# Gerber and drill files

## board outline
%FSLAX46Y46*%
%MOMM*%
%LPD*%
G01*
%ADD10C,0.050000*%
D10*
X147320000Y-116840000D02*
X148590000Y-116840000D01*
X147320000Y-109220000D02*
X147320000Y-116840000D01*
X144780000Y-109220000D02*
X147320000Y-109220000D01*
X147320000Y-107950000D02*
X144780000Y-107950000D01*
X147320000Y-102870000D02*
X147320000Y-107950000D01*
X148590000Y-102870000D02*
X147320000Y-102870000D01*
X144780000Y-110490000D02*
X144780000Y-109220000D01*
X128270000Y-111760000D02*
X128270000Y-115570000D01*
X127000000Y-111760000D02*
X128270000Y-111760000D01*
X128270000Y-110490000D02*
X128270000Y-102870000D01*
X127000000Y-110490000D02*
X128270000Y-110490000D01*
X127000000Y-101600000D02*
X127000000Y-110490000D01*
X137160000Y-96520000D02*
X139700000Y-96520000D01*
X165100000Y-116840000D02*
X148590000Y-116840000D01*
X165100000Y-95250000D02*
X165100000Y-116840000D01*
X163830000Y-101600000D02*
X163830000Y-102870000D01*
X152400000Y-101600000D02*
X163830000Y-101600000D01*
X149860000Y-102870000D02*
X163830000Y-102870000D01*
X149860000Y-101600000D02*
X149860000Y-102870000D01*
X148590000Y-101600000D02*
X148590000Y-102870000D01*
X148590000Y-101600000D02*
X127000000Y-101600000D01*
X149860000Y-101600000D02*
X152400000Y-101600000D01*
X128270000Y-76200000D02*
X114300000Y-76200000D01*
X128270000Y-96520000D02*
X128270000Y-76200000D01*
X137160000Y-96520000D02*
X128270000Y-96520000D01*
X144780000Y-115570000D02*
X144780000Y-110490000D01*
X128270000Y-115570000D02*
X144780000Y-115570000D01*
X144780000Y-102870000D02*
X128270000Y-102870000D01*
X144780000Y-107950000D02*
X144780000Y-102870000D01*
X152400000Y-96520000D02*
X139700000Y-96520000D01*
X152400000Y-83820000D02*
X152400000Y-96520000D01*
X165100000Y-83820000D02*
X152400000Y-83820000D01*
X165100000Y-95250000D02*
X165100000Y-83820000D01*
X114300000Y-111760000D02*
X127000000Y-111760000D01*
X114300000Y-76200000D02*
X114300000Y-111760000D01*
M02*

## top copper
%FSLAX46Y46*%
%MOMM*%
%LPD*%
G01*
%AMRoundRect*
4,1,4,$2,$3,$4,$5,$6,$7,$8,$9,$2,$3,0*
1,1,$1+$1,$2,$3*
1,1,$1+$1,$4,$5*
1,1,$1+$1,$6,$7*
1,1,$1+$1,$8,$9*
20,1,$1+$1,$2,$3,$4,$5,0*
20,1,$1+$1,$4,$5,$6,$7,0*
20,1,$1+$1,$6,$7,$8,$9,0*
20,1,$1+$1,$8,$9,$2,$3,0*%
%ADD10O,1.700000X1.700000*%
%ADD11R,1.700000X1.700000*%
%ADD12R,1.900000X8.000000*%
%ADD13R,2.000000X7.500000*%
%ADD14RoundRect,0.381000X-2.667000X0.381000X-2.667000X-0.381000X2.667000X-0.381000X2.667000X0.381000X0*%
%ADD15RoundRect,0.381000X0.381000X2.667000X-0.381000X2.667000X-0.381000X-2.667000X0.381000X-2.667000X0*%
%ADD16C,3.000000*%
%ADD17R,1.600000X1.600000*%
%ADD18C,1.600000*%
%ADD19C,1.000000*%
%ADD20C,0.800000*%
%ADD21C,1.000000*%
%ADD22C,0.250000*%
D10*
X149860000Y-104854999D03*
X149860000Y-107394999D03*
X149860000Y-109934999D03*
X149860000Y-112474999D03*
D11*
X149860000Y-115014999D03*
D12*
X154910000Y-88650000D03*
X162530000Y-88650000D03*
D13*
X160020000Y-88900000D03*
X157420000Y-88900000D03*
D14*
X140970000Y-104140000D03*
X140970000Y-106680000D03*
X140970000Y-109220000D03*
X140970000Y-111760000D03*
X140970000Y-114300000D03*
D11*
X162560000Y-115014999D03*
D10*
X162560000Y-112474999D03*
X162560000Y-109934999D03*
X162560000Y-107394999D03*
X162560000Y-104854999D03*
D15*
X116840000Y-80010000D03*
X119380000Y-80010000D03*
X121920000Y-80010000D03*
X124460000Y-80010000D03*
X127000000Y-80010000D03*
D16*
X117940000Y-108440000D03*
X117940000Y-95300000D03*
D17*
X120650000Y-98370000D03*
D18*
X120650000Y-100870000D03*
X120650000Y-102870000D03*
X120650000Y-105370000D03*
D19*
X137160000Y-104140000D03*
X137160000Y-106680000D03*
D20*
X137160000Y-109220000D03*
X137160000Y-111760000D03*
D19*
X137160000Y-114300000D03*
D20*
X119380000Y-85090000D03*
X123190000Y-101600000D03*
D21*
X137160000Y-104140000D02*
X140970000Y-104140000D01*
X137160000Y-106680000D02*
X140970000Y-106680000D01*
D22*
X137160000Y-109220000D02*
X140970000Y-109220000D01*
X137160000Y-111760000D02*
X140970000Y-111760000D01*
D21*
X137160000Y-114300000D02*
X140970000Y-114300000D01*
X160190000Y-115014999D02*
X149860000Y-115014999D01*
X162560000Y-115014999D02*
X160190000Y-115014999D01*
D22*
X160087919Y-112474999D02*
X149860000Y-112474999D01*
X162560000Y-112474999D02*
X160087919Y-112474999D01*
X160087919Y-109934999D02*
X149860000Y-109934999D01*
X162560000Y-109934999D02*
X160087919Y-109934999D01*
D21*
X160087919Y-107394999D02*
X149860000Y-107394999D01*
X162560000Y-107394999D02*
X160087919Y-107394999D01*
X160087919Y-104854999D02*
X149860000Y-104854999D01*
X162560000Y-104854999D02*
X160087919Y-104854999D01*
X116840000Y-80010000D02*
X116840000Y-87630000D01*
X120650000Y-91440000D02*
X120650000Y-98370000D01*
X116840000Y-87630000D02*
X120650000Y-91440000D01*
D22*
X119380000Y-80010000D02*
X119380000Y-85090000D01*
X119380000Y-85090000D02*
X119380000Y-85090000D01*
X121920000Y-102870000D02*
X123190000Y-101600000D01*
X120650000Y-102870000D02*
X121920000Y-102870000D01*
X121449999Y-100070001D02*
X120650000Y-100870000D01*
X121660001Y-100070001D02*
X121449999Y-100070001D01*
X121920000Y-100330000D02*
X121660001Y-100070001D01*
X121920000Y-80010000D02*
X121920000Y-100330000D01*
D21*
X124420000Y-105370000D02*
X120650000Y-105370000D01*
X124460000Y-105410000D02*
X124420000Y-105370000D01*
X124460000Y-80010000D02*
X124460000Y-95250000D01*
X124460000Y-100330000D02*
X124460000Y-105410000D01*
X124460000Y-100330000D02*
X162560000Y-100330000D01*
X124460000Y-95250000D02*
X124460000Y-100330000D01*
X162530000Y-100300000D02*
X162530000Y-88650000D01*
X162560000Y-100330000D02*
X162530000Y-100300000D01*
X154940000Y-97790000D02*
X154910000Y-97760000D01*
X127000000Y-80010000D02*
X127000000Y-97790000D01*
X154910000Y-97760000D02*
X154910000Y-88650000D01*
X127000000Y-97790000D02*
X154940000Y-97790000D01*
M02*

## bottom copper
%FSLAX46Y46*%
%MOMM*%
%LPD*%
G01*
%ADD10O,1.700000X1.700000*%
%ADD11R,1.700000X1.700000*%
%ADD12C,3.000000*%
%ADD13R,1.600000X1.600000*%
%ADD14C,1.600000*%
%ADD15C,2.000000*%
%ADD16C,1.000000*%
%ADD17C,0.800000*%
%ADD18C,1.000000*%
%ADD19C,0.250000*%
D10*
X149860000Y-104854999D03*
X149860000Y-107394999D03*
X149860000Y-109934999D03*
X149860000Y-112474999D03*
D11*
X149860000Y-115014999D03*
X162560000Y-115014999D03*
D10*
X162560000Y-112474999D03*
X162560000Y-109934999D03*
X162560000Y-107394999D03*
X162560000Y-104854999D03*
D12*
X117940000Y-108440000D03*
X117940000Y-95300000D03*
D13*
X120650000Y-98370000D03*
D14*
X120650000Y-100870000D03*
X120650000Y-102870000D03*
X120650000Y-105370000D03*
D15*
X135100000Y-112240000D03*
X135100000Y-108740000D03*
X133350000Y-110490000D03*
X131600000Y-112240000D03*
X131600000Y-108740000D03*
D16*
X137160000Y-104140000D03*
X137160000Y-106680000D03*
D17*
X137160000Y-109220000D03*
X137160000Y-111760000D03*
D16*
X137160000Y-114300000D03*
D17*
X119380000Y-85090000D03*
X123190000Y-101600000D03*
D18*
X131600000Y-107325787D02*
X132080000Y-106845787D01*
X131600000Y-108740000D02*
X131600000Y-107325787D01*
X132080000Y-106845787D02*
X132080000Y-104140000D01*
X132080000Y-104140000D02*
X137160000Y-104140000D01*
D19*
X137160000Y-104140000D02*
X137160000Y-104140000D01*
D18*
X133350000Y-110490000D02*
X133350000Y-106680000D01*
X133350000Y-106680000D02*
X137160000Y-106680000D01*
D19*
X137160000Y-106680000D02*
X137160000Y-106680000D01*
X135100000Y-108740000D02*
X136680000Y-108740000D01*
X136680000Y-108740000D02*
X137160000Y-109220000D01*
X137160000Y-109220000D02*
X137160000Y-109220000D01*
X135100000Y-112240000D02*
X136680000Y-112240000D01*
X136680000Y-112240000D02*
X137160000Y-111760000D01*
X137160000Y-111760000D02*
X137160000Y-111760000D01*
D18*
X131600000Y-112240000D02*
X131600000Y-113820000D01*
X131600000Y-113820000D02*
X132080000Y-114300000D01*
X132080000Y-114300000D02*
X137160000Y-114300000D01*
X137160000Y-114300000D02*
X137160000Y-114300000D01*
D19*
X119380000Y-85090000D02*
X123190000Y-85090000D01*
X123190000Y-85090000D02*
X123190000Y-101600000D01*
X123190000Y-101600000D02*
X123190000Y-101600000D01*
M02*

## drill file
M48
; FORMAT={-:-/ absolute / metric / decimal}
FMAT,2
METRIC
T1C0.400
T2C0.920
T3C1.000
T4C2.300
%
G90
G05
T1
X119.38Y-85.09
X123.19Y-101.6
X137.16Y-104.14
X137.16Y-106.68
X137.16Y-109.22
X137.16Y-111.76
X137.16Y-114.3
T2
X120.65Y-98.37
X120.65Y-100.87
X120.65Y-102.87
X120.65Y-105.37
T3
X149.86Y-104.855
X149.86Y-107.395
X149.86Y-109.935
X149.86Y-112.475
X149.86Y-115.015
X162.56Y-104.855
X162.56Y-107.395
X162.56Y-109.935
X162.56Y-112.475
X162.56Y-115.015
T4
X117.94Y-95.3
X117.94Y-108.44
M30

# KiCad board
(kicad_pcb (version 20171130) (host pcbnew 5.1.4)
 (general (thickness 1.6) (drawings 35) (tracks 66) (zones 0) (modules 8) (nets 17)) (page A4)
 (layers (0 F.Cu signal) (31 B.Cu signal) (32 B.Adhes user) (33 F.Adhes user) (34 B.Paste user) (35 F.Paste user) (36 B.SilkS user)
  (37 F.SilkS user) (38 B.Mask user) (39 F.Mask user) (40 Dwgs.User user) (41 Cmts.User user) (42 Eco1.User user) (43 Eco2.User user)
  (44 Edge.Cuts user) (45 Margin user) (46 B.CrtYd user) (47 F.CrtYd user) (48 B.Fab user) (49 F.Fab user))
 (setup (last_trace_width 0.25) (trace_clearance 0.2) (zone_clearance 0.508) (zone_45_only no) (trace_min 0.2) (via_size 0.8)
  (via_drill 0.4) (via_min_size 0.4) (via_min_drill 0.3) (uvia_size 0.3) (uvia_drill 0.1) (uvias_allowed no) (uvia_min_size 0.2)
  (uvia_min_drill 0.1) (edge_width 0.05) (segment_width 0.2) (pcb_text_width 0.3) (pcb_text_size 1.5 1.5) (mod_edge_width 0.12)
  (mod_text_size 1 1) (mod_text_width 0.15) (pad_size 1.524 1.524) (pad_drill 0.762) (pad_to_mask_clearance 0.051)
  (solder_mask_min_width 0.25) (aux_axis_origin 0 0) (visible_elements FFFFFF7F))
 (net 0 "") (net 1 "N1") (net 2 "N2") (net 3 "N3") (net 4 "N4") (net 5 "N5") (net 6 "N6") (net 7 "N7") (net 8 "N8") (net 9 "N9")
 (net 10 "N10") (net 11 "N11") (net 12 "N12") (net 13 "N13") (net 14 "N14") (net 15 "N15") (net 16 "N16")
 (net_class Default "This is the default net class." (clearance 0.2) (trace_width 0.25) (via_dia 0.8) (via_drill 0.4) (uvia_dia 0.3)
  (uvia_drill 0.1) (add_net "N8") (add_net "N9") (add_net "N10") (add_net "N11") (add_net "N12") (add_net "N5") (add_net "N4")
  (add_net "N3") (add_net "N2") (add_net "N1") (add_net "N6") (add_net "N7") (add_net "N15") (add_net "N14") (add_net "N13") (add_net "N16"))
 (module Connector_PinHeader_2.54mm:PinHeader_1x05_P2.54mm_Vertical (layer F.Cu) (at 149.86 115.014999 180)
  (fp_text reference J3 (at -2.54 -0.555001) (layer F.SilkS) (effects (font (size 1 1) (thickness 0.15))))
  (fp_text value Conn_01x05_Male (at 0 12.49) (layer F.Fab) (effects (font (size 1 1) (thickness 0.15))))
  (pad 5 thru_hole oval (at 0 10.16 180) (size 1.7 1.7) (drill 1) (layers *.Cu *.Mask) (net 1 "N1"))
  (pad 4 thru_hole oval (at 0 7.62 180) (size 1.7 1.7) (drill 1) (layers *.Cu *.Mask) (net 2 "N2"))
  (pad 3 thru_hole oval (at 0 5.08 180) (size 1.7 1.7) (drill 1) (layers *.Cu *.Mask) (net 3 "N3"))
  (pad 2 thru_hole oval (at 0 2.54 180) (size 1.7 1.7) (drill 1) (layers *.Cu *.Mask) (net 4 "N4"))
  (pad 1 thru_hole rect (at 0 0 180) (size 1.7 1.7) (drill 1) (layers *.Cu *.Mask) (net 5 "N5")))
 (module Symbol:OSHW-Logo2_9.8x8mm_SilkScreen (layer F.Cu) (at 132.08 109.22 90)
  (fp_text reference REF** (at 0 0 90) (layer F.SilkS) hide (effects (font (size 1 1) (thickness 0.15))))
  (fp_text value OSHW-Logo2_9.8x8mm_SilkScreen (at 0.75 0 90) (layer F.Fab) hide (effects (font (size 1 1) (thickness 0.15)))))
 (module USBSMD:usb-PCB (layer F.Cu) (at 158.72 83.75 180)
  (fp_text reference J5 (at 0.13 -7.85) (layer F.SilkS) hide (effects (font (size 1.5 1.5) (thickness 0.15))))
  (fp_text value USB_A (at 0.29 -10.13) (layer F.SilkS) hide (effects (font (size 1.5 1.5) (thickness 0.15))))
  (pad 1 connect rect (at 3.81 -4.9 180) (size 1.9 8) (layers F.Cu F.Mask) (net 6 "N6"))
  (pad 4 connect rect (at -3.81 -4.9 180) (size 1.9 8) (layers F.Cu F.Mask) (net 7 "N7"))
  (pad 3 connect rect (at -1.3 -5.15 180) (size 2 7.5) (layers F.Cu F.Mask))
  (pad 2 connect rect (at 1.3 -5.15 180) (size 2 7.5) (layers F.Cu F.Mask)))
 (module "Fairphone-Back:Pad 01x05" (layer F.Cu) (at 140.97 109.22 270)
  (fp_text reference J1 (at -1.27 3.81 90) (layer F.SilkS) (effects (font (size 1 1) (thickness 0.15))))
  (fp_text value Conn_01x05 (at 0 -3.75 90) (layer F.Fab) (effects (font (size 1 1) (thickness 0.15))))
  (pad 1 smd roundrect (at -5.08 0 270) (size 1.524 6.096) (layers F.Cu F.Paste F.Mask) (roundrect_rratio 0.25) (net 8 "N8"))
  (pad 2 smd roundrect (at -2.54 0 270) (size 1.524 6.096) (layers F.Cu F.Paste F.Mask) (roundrect_rratio 0.25) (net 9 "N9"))
  (pad 3 smd roundrect (at 0 0 270) (size 1.524 6.096) (layers F.Cu F.Paste F.Mask) (roundrect_rratio 0.25) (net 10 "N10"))
  (pad 4 smd roundrect (at 2.54 0 270) (size 1.524 6.096) (layers F.Cu F.Paste F.Mask) (roundrect_rratio 0.25) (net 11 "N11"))
  (pad 5 smd roundrect (at 5.08 0 270) (size 1.524 6.096) (layers F.Cu F.Paste F.Mask) (roundrect_rratio 0.25) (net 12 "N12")))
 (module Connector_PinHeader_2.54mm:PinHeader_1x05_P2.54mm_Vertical (layer F.Cu) (at 162.56 115.014999 180)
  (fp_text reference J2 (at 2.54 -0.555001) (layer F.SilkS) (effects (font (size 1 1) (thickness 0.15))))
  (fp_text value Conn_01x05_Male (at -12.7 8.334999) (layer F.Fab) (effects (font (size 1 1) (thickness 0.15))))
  (pad 1 thru_hole rect (at 0 0 180) (size 1.7 1.7) (drill 1) (layers *.Cu *.Mask) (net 5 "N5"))
  (pad 2 thru_hole oval (at 0 2.54 180) (size 1.7 1.7) (drill 1) (layers *.Cu *.Mask) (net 4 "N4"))
  (pad 3 thru_hole oval (at 0 5.08 180) (size 1.7 1.7) (drill 1) (layers *.Cu *.Mask) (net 3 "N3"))
  (pad 4 thru_hole oval (at 0 7.62 180) (size 1.7 1.7) (drill 1) (layers *.Cu *.Mask) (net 2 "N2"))
  (pad 5 thru_hole oval (at 0 10.16 180) (size 1.7 1.7) (drill 1) (layers *.Cu *.Mask) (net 1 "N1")))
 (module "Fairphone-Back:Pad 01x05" (layer F.Cu) (at 121.92 80.01 180)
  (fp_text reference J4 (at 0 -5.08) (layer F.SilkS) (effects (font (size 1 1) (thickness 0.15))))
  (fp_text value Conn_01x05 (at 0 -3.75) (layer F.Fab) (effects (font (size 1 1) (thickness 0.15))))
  (pad 5 smd roundrect (at 5.08 0 180) (size 1.524 6.096) (layers F.Cu F.Paste F.Mask) (roundrect_rratio 0.25) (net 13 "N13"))
  (pad 4 smd roundrect (at 2.54 0 180) (size 1.524 6.096) (layers F.Cu F.Paste F.Mask) (roundrect_rratio 0.25) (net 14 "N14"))
  (pad 3 smd roundrect (at 0 0 180) (size 1.524 6.096) (layers F.Cu F.Paste F.Mask) (roundrect_rratio 0.25) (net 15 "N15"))
  (pad 2 smd roundrect (at -2.54 0 180) (size 1.524 6.096) (layers F.Cu F.Paste F.Mask) (roundrect_rratio 0.25) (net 7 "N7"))
  (pad 1 smd roundrect (at -5.08 0 180) (size 1.524 6.096) (layers F.Cu F.Paste F.Mask) (roundrect_rratio 0.25) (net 6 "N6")))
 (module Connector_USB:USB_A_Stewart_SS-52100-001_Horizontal (layer F.Cu) (at 120.65 98.37 270)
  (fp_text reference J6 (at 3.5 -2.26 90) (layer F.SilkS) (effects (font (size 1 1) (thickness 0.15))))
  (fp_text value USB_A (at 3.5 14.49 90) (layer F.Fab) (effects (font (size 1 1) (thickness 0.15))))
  (pad 5 thru_hole circle (at 10.07 2.71 270) (size 3 3) (drill 2.3) (layers *.Cu *.Mask) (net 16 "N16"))
  (pad 5 thru_hole circle (at -3.07 2.71 270) (size 3 3) (drill 2.3) (layers *.Cu *.Mask) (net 16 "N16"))
  (pad 1 thru_hole rect (at 0 0 270) (size 1.6 1.6) (drill 0.92) (layers *.Cu *.Mask) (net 13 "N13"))
  (pad 2 thru_hole circle (at 2.5 0 270) (size 1.6 1.6) (drill 0.92) (layers *.Cu *.Mask) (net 15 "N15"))
  (pad 3 thru_hole circle (at 4.5 0 270) (size 1.6 1.6) (drill 0.92) (layers *.Cu *.Mask) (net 14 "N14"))
  (pad 4 thru_hole circle (at 7 0 270) (size 1.6 1.6) (drill 0.92) (layers *.Cu *.Mask) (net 7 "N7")))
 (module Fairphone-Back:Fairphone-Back (layer F.Cu) (at 133.35 110.49 90)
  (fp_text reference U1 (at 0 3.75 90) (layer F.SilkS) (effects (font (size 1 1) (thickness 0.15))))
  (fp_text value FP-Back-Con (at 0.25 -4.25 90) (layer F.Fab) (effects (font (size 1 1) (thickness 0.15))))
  (pad 4 connect circle (at -1.75 1.75 90) (size 2 2) (layers B.Cu B.Mask) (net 11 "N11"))
  (pad 5 connect circle (at 1.75 1.75 90) (size 2 2) (layers B.Cu B.Mask) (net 10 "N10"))
  (pad 3 connect circle (at 0 0 90) (size 2 2) (layers B.Cu B.Mask) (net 9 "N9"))
  (pad 1 connect circle (at -1.75 -1.75 90) (size 2 2) (layers B.Cu B.Mask) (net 12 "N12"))
  (pad 2 connect circle (at 1.75 -1.75 90) (size 2 2) (layers B.Cu B.Mask) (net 8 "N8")))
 (gr_line (start 147.32 116.84) (end 148.59 116.84) (layer Edge.Cuts) (width 0.05))
 (gr_line (start 147.32 109.22) (end 147.32 116.84) (layer Edge.Cuts) (width 0.05))
 (gr_line (start 144.78 109.22) (end 147.32 109.22) (layer Edge.Cuts) (width 0.05))
 (gr_line (start 147.32 107.95) (end 144.78 107.95) (layer Edge.Cuts) (width 0.05))
 (gr_line (start 147.32 102.87) (end 147.32 107.95) (layer Edge.Cuts) (width 0.05))
 (gr_line (start 148.59 102.87) (end 147.32 102.87) (layer Edge.Cuts) (width 0.05))
 (gr_line (start 144.78 110.49) (end 144.78 109.22) (layer Edge.Cuts) (width 0.05))
 (gr_line (start 128.27 111.76) (end 128.27 115.57) (layer Edge.Cuts) (width 0.05))
 (gr_line (start 127 111.76) (end 128.27 111.76) (layer Edge.Cuts) (width 0.05))
 (gr_line (start 128.27 110.49) (end 128.27 102.87) (layer Edge.Cuts) (width 0.05))
 (gr_line (start 127 110.49) (end 128.27 110.49) (layer Edge.Cuts) (width 0.05))
 (gr_line (start 127 101.6) (end 127 110.49) (layer Edge.Cuts) (width 0.05))
 (gr_line (start 137.16 96.52) (end 139.7 96.52) (layer Edge.Cuts) (width 0.05))
 (gr_line (start 165.1 116.84) (end 148.59 116.84) (layer Edge.Cuts) (width 0.05))
 (gr_line (start 165.1 95.25) (end 165.1 116.84) (layer Edge.Cuts) (width 0.05))
 (gr_line (start 163.83 101.6) (end 163.83 102.87) (layer Edge.Cuts) (width 0.05))
 (gr_line (start 152.4 101.6) (end 163.83 101.6) (layer Edge.Cuts) (width 0.05))
 (gr_line (start 149.86 102.87) (end 163.83 102.87) (layer Edge.Cuts) (width 0.05))
 (gr_line (start 149.86 101.6) (end 149.86 102.87) (layer Edge.Cuts) (width 0.05))
 (gr_line (start 148.59 101.6) (end 148.59 102.87) (layer Edge.Cuts) (width 0.05))
 (gr_line (start 148.59 101.6) (end 127 101.6) (layer Edge.Cuts) (width 0.05))
 (gr_line (start 149.86 101.6) (end 152.4 101.6) (layer Edge.Cuts) (width 0.05))
 (gr_line (start 128.27 76.2) (end 114.3 76.2) (layer Edge.Cuts) (width 0.05))
 (gr_line (start 128.27 96.52) (end 128.27 76.2) (layer Edge.Cuts) (width 0.05))
 (gr_line (start 137.16 96.52) (end 128.27 96.52) (layer Edge.Cuts) (width 0.05))
 (gr_line (start 144.78 115.57) (end 144.78 110.49) (layer Edge.Cuts) (width 0.05))
 (gr_line (start 128.27 115.57) (end 144.78 115.57) (layer Edge.Cuts) (width 0.05))
 (gr_line (start 144.78 102.87) (end 128.27 102.87) (layer Edge.Cuts) (width 0.05))
 (gr_line (start 144.78 107.95) (end 144.78 102.87) (layer Edge.Cuts) (width 0.05))
 (gr_line (start 152.4 96.52) (end 139.7 96.52) (layer Edge.Cuts) (width 0.05))
 (gr_line (start 152.4 83.82) (end 152.4 96.52) (layer Edge.Cuts) (width 0.05))
 (gr_line (start 165.1 83.82) (end 152.4 83.82) (layer Edge.Cuts) (width 0.05))
 (gr_line (start 165.1 95.25) (end 165.1 83.82) (layer Edge.Cuts) (width 0.05))
 (gr_line (start 114.3 111.76) (end 127 111.76) (layer Edge.Cuts) (width 0.05))
 (gr_line (start 114.3 76.2) (end 114.3 111.76) (layer Edge.Cuts) (width 0.05))
 (segment (start 131.6 107.325787) (end 132.08 106.845787) (width 1) (layer B.Cu) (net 8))
 (segment (start 131.6 108.74) (end 131.6 107.325787) (width 1) (layer B.Cu) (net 8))
 (segment (start 132.08 106.845787) (end 132.08 104.14) (width 1) (layer B.Cu) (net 8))
 (segment (start 132.08 104.14) (end 137.16 104.14) (width 1) (layer B.Cu) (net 8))
 (segment (start 137.16 104.14) (end 137.16 104.14) (width 0.25) (layer B.Cu) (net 8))
 (via (at 137.16 104.14) (size 1) (drill 0.4) (layers F.Cu B.Cu) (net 8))
 (segment (start 137.16 104.14) (end 140.97 104.14) (width 1) (layer F.Cu) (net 8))
 (segment (start 133.35 110.49) (end 133.35 106.68) (width 1) (layer B.Cu) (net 9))
 (segment (start 133.35 106.68) (end 137.16 106.68) (width 1) (layer B.Cu) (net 9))
 (segment (start 137.16 106.68) (end 137.16 106.68) (width 0.25) (layer B.Cu) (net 9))
 (via (at 137.16 106.68) (size 1) (drill 0.4) (layers F.Cu B.Cu) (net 9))
 (segment (start 137.16 106.68) (end 140.97 106.68) (width 1) (layer F.Cu) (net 9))
 (segment (start 135.1 108.74) (end 136.68 108.74) (width 0.25) (layer B.Cu) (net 10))
 (segment (start 136.68 108.74) (end 137.16 109.22) (width 0.25) (layer B.Cu) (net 10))
 (segment (start 137.16 109.22) (end 137.16 109.22) (width 0.25) (layer B.Cu) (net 10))
 (via (at 137.16 109.22) (size 0.8) (drill 0.4) (layers F.Cu B.Cu) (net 10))
 (segment (start 137.16 109.22) (end 140.97 109.22) (width 0.25) (layer F.Cu) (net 10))
 (segment (start 135.1 112.24) (end 136.68 112.24) (width 0.25) (layer B.Cu) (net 11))
 (segment (start 136.68 112.24) (end 137.16 111.76) (width 0.25) (layer B.Cu) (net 11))
 (segment (start 137.16 111.76) (end 137.16 111.76) (width 0.25) (layer B.Cu) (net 11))
 (via (at 137.16 111.76) (size 0.8) (drill 0.4) (layers F.Cu B.Cu) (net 11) (status 1000000))
 (segment (start 137.16 111.76) (end 140.97 111.76) (width 0.25) (layer F.Cu) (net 11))
 (segment (start 131.6 112.24) (end 131.6 113.82) (width 1) (layer B.Cu) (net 12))
 (segment (start 131.6 113.82) (end 132.08 114.3) (width 1) (layer B.Cu) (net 12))
 (segment (start 132.08 114.3) (end 137.16 114.3) (width 1) (layer B.Cu) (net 12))
 (segment (start 137.16 114.3) (end 137.16 114.3) (width 1) (layer B.Cu) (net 12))
 (via (at 137.16 114.3) (size 1) (drill 0.4) (layers F.Cu B.Cu) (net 12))
 (segment (start 137.16 114.3) (end 140.97 114.3) (width 1) (layer F.Cu) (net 12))
 (segment (start 160.19 115.014999) (end 149.86 115.014999) (width 1) (layer F.Cu) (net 5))
 (segment (start 162.56 115.014999) (end 160.19 115.014999) (width 1) (layer F.Cu) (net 5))
 (segment (start 160.087919 112.474999) (end 149.86 112.474999) (width 0.25) (layer F.Cu) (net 4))
 (segment (start 162.56 112.474999) (end 160.087919 112.474999) (width 0.25) (layer F.Cu) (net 4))
 (segment (start 160.087919 109.934999) (end 149.86 109.934999) (width 0.25) (layer F.Cu) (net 3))
 (segment (start 162.56 109.934999) (end 160.087919 109.934999) (width 0.25) (layer F.Cu) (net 3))
 (segment (start 160.087919 107.394999) (end 149.86 107.394999) (width 1) (layer F.Cu) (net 2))
 (segment (start 162.56 107.394999) (end 160.087919 107.394999) (width 1) (layer F.Cu) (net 2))
 (segment (start 160.087919 104.854999) (end 149.86 104.854999) (width 1) (layer F.Cu) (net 1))
 (segment (start 162.56 104.854999) (end 160.087919 104.854999) (width 1) (layer F.Cu) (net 1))
 (segment (start 116.84 80.01) (end 116.84 87.63) (width 1) (layer F.Cu) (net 13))
 (segment (start 120.65 91.44) (end 120.65 98.37) (width 1) (layer F.Cu) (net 13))
 (segment (start 116.84 87.63) (end 120.65 91.44) (width 1) (layer F.Cu) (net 13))
 (segment (start 119.38 80.01) (end 119.38 85.09) (width 0.25) (layer F.Cu) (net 14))
 (segment (start 119.38 85.09) (end 119.38 85.09) (width 0.25) (layer F.Cu) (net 14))
 (via (at 119.38 85.09) (size 0.8) (drill 0.4) (layers F.Cu B.Cu) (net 14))
 (segment (start 119.38 85.09) (end 123.19 85.09) (width 0.25) (layer B.Cu) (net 14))
 (segment (start 123.19 85.09) (end 123.19 101.6) (width 0.25) (layer B.Cu) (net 14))
 (segment (start 123.19 101.6) (end 123.19 101.6) (width 0.25) (layer B.Cu) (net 14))
 (via (at 123.19 101.6) (size 0.8) (drill 0.4) (layers F.Cu B.Cu) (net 14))
 (segment (start 121.92 102.87) (end 123.19 101.6) (width 0.25) (layer F.Cu) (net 14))
 (segment (start 120.65 102.87) (end 121.92 102.87) (width 0.25) (layer F.Cu) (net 14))
 (segment (start 121.449999 100.070001) (end 120.65 100.87) (width 0.25) (layer F.Cu) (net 15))
 (segment (start 121.660001 100.070001) (end 121.449999 100.070001) (width 0.25) (layer F.Cu) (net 15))
 (segment (start 121.92 100.33) (end 121.660001 100.070001) (width 0.25) (layer F.Cu) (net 15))
 (segment (start 121.92 80.01) (end 121.92 100.33) (width 0.25) (layer F.Cu) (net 15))
 (segment (start 124.42 105.37) (end 120.65 105.37) (width 1) (layer F.Cu) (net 7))
 (segment (start 124.46 105.41) (end 124.42 105.37) (width 1) (layer F.Cu) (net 7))
 (segment (start 124.46 80.01) (end 124.46 95.25) (width 1) (layer F.Cu) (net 7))
 (segment (start 124.46 100.33) (end 124.46 105.41) (width 1) (layer F.Cu) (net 7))
 (segment (start 124.46 100.33) (end 162.56 100.33) (width 1) (layer F.Cu) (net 7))
 (segment (start 124.46 95.25) (end 124.46 100.33) (width 1) (layer F.Cu) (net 7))
 (segment (start 162.53 100.3) (end 162.53 88.65) (width 1) (layer F.Cu) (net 7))
 (segment (start 162.56 100.33) (end 162.53 100.3) (width 1) (layer F.Cu) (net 7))
 (segment (start 154.94 97.79) (end 154.91 97.76) (width 1) (layer F.Cu) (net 6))
 (segment (start 127 80.01) (end 127 97.79) (width 1) (layer F.Cu) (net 6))
 (segment (start 154.91 97.76) (end 154.91 88.65) (width 1) (layer F.Cu) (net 6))
 (segment (start 127 97.79) (end 154.94 97.79) (width 1) (layer F.Cu) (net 6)))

